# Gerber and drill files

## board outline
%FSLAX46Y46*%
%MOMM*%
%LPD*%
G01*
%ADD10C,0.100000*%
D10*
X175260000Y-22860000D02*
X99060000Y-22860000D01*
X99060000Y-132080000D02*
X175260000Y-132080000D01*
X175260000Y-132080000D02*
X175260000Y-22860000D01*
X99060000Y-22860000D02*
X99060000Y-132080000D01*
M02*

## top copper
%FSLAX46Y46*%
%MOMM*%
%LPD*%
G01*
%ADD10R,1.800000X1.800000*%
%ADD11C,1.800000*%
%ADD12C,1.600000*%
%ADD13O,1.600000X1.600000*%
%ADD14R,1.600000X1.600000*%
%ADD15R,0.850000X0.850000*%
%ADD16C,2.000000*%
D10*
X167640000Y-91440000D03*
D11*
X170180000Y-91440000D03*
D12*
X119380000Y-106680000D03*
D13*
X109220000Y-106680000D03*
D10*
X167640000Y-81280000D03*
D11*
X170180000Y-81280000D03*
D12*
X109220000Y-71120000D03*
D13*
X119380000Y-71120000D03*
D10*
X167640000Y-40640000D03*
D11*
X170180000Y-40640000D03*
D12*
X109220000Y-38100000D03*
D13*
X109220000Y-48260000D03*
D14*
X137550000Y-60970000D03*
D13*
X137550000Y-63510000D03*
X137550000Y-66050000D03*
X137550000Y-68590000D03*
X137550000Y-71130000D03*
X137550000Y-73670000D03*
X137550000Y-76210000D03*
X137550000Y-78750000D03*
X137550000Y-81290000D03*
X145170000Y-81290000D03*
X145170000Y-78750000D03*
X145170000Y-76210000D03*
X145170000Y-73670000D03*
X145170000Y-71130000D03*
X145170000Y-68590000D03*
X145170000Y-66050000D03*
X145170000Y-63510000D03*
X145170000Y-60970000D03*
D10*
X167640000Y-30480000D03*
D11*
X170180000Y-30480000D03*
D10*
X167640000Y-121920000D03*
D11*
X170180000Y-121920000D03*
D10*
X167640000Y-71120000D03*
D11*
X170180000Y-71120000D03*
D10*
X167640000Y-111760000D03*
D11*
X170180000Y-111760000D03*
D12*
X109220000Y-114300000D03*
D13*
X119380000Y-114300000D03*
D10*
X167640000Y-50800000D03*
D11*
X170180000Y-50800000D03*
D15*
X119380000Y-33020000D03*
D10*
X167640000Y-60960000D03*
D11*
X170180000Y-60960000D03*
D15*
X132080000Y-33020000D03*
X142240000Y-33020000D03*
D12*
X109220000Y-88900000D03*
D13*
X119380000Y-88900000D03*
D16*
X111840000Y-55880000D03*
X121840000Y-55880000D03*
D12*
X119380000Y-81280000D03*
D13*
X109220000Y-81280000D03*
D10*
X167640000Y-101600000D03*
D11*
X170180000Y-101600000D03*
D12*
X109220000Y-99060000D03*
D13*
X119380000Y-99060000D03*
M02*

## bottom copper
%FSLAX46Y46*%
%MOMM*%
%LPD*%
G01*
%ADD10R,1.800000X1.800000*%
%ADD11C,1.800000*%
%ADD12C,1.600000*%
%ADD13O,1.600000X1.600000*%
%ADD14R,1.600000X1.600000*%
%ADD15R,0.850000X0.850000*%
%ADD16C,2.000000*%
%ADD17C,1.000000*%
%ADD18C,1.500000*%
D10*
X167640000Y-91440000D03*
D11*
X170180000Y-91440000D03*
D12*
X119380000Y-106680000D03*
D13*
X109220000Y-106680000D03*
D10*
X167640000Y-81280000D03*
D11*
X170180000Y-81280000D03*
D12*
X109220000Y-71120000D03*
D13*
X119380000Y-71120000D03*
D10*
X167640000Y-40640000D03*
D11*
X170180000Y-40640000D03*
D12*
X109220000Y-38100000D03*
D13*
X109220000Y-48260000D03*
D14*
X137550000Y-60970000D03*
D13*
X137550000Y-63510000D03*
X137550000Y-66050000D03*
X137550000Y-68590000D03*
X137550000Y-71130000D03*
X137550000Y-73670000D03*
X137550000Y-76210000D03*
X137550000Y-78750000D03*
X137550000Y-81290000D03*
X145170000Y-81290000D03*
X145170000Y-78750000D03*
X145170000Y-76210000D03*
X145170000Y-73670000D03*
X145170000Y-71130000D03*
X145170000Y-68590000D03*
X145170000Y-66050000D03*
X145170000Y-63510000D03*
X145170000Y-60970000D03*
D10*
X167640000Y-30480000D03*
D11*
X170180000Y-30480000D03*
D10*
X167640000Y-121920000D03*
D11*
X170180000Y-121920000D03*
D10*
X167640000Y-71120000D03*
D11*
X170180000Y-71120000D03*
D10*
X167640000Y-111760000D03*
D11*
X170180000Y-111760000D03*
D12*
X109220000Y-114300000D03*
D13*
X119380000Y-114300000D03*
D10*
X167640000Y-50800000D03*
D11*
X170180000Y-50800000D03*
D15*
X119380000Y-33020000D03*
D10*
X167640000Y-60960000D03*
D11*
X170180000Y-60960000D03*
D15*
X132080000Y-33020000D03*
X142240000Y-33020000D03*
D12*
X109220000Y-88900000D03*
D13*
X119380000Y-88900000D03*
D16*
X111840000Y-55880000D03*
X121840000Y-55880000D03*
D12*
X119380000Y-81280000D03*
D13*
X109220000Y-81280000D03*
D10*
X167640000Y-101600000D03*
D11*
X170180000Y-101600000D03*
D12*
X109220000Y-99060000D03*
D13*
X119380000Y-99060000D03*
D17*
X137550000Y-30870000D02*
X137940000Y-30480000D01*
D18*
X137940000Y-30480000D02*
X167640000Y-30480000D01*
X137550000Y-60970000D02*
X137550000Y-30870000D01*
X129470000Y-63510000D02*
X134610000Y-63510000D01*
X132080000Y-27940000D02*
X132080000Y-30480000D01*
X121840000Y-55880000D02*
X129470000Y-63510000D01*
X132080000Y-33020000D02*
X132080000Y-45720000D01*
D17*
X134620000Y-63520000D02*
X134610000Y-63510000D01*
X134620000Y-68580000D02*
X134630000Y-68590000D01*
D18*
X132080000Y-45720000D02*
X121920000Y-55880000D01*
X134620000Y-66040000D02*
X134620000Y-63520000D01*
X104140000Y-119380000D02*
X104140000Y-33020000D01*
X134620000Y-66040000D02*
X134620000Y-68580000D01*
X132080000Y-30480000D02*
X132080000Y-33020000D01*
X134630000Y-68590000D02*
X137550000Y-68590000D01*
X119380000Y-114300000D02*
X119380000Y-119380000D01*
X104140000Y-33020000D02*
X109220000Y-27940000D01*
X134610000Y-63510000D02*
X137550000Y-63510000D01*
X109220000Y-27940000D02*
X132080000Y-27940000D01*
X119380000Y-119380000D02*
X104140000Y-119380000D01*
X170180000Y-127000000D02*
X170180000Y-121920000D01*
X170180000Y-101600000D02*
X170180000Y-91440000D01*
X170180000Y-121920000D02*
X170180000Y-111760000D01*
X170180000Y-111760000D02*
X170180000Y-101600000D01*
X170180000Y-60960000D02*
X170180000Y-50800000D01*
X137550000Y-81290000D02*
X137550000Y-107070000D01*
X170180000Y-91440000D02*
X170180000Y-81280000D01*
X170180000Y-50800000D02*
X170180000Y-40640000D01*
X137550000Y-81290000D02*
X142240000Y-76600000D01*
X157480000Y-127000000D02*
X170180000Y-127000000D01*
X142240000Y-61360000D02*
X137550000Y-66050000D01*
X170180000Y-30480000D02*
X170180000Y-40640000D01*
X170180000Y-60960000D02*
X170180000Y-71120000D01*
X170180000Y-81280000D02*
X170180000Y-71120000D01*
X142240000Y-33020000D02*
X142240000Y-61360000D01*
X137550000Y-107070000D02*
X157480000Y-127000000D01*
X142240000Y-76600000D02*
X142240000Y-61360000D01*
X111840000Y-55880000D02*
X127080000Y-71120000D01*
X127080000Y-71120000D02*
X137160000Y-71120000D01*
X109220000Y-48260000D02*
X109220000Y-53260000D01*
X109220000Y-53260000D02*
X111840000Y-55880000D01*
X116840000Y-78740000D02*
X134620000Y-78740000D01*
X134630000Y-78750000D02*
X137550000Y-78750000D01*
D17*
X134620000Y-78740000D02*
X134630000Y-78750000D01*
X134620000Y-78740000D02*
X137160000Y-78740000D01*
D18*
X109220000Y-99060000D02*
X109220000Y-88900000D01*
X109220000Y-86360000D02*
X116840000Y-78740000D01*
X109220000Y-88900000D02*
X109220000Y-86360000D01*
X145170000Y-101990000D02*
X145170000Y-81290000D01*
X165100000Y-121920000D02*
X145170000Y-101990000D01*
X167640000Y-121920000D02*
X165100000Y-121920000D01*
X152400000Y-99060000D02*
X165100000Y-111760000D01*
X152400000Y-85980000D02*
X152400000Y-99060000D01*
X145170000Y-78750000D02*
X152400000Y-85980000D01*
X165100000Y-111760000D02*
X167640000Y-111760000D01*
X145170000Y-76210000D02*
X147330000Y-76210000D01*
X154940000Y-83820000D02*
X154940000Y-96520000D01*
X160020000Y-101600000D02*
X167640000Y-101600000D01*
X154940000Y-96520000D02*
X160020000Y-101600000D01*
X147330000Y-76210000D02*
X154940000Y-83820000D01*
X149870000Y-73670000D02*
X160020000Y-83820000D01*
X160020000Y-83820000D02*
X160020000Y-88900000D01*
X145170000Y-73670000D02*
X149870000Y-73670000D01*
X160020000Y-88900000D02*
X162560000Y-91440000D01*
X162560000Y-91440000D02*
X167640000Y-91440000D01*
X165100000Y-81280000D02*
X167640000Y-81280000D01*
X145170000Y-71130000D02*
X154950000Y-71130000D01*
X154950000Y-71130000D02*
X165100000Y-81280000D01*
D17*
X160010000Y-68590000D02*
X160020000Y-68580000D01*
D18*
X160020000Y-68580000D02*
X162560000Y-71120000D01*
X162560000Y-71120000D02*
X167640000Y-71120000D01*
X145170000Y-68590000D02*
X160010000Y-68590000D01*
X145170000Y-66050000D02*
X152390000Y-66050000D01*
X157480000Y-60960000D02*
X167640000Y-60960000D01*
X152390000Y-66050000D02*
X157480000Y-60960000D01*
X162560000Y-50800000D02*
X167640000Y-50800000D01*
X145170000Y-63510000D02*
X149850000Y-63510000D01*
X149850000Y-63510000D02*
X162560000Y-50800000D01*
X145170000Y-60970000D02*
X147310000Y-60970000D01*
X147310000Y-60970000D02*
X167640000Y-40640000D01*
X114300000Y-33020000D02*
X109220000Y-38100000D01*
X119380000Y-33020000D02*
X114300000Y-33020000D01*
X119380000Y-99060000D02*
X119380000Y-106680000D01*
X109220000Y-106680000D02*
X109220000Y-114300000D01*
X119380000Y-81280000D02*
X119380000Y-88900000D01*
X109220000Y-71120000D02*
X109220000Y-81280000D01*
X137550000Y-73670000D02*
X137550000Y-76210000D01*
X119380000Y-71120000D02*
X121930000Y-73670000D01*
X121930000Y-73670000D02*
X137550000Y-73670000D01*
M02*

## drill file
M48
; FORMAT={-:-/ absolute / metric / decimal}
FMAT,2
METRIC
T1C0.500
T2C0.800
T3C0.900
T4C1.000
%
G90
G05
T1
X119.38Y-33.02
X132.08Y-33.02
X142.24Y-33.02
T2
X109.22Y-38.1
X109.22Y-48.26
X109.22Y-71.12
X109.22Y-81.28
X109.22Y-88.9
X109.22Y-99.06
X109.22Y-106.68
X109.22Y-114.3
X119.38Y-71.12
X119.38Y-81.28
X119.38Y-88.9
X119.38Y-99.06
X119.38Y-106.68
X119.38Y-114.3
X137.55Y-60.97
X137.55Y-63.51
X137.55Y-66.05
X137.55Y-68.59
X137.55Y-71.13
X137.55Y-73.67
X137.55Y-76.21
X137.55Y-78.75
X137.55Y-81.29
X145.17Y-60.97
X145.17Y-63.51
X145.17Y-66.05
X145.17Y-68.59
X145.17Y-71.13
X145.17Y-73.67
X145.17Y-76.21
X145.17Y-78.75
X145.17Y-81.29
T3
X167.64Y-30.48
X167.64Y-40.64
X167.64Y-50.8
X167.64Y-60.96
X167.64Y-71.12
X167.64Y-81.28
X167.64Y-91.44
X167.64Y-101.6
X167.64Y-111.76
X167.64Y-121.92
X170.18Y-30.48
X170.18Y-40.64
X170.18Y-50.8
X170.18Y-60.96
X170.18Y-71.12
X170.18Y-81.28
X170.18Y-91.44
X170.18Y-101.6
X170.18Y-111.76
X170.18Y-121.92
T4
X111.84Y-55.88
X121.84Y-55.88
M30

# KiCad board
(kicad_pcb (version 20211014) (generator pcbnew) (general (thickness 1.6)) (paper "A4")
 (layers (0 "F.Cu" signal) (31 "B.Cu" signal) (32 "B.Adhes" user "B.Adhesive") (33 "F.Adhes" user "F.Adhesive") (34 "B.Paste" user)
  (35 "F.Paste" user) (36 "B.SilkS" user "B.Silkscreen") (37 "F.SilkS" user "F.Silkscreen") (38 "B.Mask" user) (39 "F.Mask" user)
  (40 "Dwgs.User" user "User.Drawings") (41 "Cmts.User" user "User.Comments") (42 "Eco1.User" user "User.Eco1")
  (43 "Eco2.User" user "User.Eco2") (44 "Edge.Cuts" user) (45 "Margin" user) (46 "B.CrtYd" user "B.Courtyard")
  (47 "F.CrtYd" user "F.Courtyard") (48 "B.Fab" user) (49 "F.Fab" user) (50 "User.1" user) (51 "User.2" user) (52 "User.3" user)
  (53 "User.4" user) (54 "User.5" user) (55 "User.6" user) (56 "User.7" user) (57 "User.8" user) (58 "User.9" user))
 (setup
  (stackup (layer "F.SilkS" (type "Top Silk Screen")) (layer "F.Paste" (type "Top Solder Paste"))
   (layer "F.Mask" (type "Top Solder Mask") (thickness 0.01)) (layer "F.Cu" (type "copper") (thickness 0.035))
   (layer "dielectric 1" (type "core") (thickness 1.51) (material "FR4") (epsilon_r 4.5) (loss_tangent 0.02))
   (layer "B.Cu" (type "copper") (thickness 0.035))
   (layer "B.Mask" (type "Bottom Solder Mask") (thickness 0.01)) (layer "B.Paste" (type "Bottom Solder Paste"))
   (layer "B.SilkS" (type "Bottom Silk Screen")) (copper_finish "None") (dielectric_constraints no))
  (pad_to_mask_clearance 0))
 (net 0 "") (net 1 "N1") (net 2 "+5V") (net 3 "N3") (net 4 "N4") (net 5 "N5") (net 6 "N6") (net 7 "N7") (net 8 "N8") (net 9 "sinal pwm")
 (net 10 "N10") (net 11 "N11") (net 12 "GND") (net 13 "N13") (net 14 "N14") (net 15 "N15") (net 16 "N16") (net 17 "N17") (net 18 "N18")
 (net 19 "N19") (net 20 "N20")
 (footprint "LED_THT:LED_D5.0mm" (layer "F.Cu") (at 167.64 91.44)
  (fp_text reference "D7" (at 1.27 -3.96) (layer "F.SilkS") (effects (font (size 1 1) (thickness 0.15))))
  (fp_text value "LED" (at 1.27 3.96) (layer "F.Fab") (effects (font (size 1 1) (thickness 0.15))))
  (pad "1" thru_hole rect (at 0 0) (size 1.8 1.8) (drill 0.9) (layers *.Cu *.Mask) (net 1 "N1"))
  (pad "2" thru_hole circle (at 2.54 0) (size 1.8 1.8) (drill 0.9) (layers *.Cu *.Mask) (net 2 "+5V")))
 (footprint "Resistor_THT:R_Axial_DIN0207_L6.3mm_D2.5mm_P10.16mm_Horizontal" (layer "F.Cu") (at 119.38 106.68 180)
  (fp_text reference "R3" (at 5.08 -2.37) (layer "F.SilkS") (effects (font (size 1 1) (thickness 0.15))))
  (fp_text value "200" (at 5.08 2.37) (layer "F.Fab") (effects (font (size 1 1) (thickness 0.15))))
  (pad "1" thru_hole circle (at 0 0 180) (size 1.6 1.6) (drill 0.8) (layers *.Cu *.Mask) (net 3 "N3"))
  (pad "2" thru_hole oval (at 10.16 0 180) (size 1.6 1.6) (drill 0.8) (layers *.Cu *.Mask) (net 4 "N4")))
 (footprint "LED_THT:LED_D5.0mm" (layer "F.Cu") (at 167.64 81.28)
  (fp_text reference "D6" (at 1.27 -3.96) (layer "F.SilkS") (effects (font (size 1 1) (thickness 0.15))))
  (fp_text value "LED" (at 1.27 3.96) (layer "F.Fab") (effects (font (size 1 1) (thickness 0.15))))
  (pad "1" thru_hole rect (at 0 0) (size 1.8 1.8) (drill 0.9) (layers *.Cu *.Mask) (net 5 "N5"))
  (pad "2" thru_hole circle (at 2.54 0) (size 1.8 1.8) (drill 0.9) (layers *.Cu *.Mask) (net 2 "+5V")))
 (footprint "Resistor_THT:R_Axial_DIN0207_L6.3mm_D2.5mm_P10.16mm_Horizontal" (layer "F.Cu") (at 109.22 71.12)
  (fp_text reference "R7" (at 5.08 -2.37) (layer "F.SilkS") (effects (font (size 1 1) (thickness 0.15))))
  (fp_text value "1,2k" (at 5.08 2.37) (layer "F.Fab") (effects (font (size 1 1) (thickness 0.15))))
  (pad "1" thru_hole circle (at 0 0) (size 1.6 1.6) (drill 0.8) (layers *.Cu *.Mask) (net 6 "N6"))
  (pad "2" thru_hole oval (at 10.16 0) (size 1.6 1.6) (drill 0.8) (layers *.Cu *.Mask) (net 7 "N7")))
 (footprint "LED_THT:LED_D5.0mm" (layer "F.Cu") (at 167.64 40.64)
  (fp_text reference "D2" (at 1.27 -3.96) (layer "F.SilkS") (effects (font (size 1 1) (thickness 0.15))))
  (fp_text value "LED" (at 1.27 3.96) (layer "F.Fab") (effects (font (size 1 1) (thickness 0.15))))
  (pad "1" thru_hole rect (at 0 0) (size 1.8 1.8) (drill 0.9) (layers *.Cu *.Mask) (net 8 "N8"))
  (pad "2" thru_hole circle (at 2.54 0) (size 1.8 1.8) (drill 0.9) (layers *.Cu *.Mask) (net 2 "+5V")))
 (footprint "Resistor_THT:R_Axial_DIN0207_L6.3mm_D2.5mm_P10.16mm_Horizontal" (layer "F.Cu") (at 109.22 38.1 -90)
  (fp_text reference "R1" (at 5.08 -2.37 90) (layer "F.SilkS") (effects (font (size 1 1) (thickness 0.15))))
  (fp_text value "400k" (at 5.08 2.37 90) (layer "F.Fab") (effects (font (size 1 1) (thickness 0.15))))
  (pad "1" thru_hole circle (at 0 0 270) (size 1.6 1.6) (drill 0.8) (layers *.Cu *.Mask) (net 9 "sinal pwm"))
  (pad "2" thru_hole oval (at 10.16 0 270) (size 1.6 1.6) (drill 0.8) (layers *.Cu *.Mask) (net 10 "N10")))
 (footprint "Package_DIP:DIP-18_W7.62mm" (layer "F.Cu") (at 137.55 60.97)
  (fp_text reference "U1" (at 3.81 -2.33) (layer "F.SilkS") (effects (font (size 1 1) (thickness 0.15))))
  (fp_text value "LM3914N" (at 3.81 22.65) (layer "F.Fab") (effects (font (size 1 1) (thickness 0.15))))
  (pad "1" thru_hole rect (at 0 0) (size 1.6 1.6) (drill 0.8) (layers *.Cu *.Mask) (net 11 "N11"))
  (pad "2" thru_hole oval (at 0 2.54) (size 1.6 1.6) (drill 0.8) (layers *.Cu *.Mask) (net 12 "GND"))
  (pad "3" thru_hole oval (at 0 5.08) (size 1.6 1.6) (drill 0.8) (layers *.Cu *.Mask) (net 2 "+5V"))
  (pad "4" thru_hole oval (at 0 7.62) (size 1.6 1.6) (drill 0.8) (layers *.Cu *.Mask) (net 12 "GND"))
  (pad "5" thru_hole oval (at 0 10.16) (size 1.6 1.6) (drill 0.8) (layers *.Cu *.Mask) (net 10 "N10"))
  (pad "6" thru_hole oval (at 0 12.7) (size 1.6 1.6) (drill 0.8) (layers *.Cu *.Mask) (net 7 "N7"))
  (pad "7" thru_hole oval (at 0 15.24) (size 1.6 1.6) (drill 0.8) (layers *.Cu *.Mask) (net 7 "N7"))
  (pad "8" thru_hole oval (at 0 17.78) (size 1.6 1.6) (drill 0.8) (layers *.Cu *.Mask) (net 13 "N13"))
  (pad "9" thru_hole oval (at 0 20.32) (size 1.6 1.6) (drill 0.8) (layers *.Cu *.Mask) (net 2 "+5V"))
  (pad "10" thru_hole oval (at 7.62 20.32) (size 1.6 1.6) (drill 0.8) (layers *.Cu *.Mask) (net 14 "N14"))
  (pad "11" thru_hole oval (at 7.62 17.78) (size 1.6 1.6) (drill 0.8) (layers *.Cu *.Mask) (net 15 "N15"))
  (pad "12" thru_hole oval (at 7.62 15.24) (size 1.6 1.6) (drill 0.8) (layers *.Cu *.Mask) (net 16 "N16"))
  (pad "13" thru_hole oval (at 7.62 12.7) (size 1.6 1.6) (drill 0.8) (layers *.Cu *.Mask) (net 1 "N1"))
  (pad "14" thru_hole oval (at 7.62 10.16) (size 1.6 1.6) (drill 0.8) (layers *.Cu *.Mask) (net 5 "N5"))
  (pad "15" thru_hole oval (at 7.62 7.62) (size 1.6 1.6) (drill 0.8) (layers *.Cu *.Mask) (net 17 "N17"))
  (pad "16" thru_hole oval (at 7.62 5.08) (size 1.6 1.6) (drill 0.8) (layers *.Cu *.Mask) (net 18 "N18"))
  (pad "17" thru_hole oval (at 7.62 2.54) (size 1.6 1.6) (drill 0.8) (layers *.Cu *.Mask) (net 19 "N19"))
  (pad "18" thru_hole oval (at 7.62 0) (size 1.6 1.6) (drill 0.8) (layers *.Cu *.Mask) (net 8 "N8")))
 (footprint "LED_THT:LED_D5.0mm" (layer "F.Cu") (at 167.64 30.48)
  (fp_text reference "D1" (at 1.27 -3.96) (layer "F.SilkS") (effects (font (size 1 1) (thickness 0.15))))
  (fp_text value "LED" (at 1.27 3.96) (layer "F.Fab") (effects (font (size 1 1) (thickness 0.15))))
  (pad "1" thru_hole rect (at 0 0) (size 1.8 1.8) (drill 0.9) (layers *.Cu *.Mask) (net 11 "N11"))
  (pad "2" thru_hole circle (at 2.54 0) (size 1.8 1.8) (drill 0.9) (layers *.Cu *.Mask) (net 2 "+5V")))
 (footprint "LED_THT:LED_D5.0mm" (layer "F.Cu") (at 167.64 121.92)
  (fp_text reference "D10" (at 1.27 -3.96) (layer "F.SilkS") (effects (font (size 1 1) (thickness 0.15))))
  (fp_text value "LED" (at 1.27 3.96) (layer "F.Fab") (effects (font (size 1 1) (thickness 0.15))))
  (pad "1" thru_hole rect (at 0 0) (size 1.8 1.8) (drill 0.9) (layers *.Cu *.Mask) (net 14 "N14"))
  (pad "2" thru_hole circle (at 2.54 0) (size 1.8 1.8) (drill 0.9) (layers *.Cu *.Mask) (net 2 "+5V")))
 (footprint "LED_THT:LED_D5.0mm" (layer "F.Cu") (at 167.64 71.12)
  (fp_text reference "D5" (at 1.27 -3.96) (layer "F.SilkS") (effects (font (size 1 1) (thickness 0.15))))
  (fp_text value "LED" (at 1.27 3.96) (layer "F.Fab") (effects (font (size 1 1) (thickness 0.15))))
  (pad "1" thru_hole rect (at 0 0) (size 1.8 1.8) (drill 0.9) (layers *.Cu *.Mask) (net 17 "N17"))
  (pad "2" thru_hole circle (at 2.54 0) (size 1.8 1.8) (drill 0.9) (layers *.Cu *.Mask) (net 2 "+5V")))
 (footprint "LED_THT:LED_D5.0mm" (layer "F.Cu") (at 167.64 111.76)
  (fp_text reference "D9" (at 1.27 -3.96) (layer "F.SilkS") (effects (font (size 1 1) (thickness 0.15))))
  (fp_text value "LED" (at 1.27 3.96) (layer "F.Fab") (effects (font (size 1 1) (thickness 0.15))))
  (pad "1" thru_hole rect (at 0 0) (size 1.8 1.8) (drill 0.9) (layers *.Cu *.Mask) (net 15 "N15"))
  (pad "2" thru_hole circle (at 2.54 0) (size 1.8 1.8) (drill 0.9) (layers *.Cu *.Mask) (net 2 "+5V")))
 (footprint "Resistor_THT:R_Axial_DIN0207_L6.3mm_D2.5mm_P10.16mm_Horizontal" (layer "F.Cu") (at 109.22 114.3)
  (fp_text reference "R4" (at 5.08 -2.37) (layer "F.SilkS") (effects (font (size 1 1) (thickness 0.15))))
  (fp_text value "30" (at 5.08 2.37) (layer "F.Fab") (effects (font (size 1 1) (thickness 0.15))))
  (pad "1" thru_hole circle (at 0 0) (size 1.6 1.6) (drill 0.8) (layers *.Cu *.Mask) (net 4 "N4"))
  (pad "2" thru_hole oval (at 10.16 0) (size 1.6 1.6) (drill 0.8) (layers *.Cu *.Mask) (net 12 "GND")))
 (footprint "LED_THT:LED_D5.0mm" (layer "F.Cu") (at 167.64 50.8)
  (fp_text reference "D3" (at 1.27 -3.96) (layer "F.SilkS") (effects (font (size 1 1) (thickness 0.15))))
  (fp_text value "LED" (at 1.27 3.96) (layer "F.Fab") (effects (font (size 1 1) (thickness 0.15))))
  (pad "1" thru_hole rect (at 0 0) (size 1.8 1.8) (drill 0.9) (layers *.Cu *.Mask) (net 19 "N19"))
  (pad "2" thru_hole circle (at 2.54 0) (size 1.8 1.8) (drill 0.9) (layers *.Cu *.Mask) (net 2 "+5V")))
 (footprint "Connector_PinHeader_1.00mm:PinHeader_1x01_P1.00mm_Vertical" (layer "F.Cu") (at 119.38 33.02)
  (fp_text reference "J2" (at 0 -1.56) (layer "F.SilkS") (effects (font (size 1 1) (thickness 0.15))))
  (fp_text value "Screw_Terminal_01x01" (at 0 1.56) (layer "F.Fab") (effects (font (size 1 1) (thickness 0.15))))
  (pad "1" thru_hole rect (at 0 0) (size 0.85 0.85) (drill 0.5) (layers *.Cu *.Mask) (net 9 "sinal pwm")))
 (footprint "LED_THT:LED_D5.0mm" (layer "F.Cu") (at 167.64 60.96)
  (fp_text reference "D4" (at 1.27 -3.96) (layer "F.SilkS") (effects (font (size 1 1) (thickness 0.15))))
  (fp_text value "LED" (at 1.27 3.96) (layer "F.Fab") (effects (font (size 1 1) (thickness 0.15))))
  (pad "1" thru_hole rect (at 0 0) (size 1.8 1.8) (drill 0.9) (layers *.Cu *.Mask) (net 18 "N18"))
  (pad "2" thru_hole circle (at 2.54 0) (size 1.8 1.8) (drill 0.9) (layers *.Cu *.Mask) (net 2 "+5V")))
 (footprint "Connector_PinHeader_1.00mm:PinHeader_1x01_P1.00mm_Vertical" (layer "F.Cu") (at 132.08 33.02)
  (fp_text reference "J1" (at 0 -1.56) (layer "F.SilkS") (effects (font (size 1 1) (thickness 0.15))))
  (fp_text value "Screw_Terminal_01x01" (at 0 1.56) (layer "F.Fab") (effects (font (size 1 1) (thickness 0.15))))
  (pad "1" thru_hole rect (at 0 0) (size 0.85 0.85) (drill 0.5) (layers *.Cu *.Mask) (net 12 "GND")))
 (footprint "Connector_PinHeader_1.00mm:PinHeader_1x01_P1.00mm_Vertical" (layer "F.Cu") (at 142.24 33.02)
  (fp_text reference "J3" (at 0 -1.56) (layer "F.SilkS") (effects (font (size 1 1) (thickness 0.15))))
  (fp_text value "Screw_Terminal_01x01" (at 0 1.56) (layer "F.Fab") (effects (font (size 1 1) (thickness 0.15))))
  (pad "1" thru_hole rect (at 0 0) (size 0.85 0.85) (drill 0.5) (layers *.Cu *.Mask) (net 2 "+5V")))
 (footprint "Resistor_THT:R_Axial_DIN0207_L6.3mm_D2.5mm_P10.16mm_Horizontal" (layer "F.Cu") (at 109.22 88.9)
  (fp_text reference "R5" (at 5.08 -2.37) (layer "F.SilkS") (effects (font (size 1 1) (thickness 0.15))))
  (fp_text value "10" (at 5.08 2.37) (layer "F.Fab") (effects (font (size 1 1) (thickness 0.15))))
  (pad "1" thru_hole circle (at 0 0) (size 1.6 1.6) (drill 0.8) (layers *.Cu *.Mask) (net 13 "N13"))
  (pad "2" thru_hole oval (at 10.16 0) (size 1.6 1.6) (drill 0.8) (layers *.Cu *.Mask) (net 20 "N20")))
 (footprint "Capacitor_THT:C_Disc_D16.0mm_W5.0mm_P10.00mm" (layer "F.Cu") (at 111.84 55.88)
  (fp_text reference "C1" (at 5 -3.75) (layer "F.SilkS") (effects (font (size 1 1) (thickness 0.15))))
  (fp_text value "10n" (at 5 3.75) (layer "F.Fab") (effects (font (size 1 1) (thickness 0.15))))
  (pad "1" thru_hole circle (at 0 0) (size 2 2) (drill 1) (layers *.Cu *.Mask) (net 10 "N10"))
  (pad "2" thru_hole circle (at 10 0) (size 2 2) (drill 1) (layers *.Cu *.Mask) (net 12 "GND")))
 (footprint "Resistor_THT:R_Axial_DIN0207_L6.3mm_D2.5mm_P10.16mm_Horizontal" (layer "F.Cu") (at 119.38 81.28 180)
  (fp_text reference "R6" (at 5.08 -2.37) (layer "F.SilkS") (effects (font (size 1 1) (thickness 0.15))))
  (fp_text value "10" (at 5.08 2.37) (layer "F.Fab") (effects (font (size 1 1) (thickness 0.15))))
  (pad "1" thru_hole circle (at 0 0 180) (size 1.6 1.6) (drill 0.8) (layers *.Cu *.Mask) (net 20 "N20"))
  (pad "2" thru_hole oval (at 10.16 0 180) (size 1.6 1.6) (drill 0.8) (layers *.Cu *.Mask) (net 6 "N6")))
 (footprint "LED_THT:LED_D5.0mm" (layer "F.Cu") (at 167.64 101.6)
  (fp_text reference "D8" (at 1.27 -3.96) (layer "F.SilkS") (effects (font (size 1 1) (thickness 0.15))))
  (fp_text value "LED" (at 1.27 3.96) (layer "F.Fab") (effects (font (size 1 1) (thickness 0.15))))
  (pad "1" thru_hole rect (at 0 0) (size 1.8 1.8) (drill 0.9) (layers *.Cu *.Mask) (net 16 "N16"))
  (pad "2" thru_hole circle (at 2.54 0) (size 1.8 1.8) (drill 0.9) (layers *.Cu *.Mask) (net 2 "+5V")))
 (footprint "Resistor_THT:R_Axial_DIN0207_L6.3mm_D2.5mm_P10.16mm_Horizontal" (layer "F.Cu") (at 109.22 99.06)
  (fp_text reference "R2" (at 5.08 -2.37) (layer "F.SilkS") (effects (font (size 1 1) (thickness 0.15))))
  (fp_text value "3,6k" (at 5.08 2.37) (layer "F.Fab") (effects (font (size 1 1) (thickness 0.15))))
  (pad "1" thru_hole circle (at 0 0) (size 1.6 1.6) (drill 0.8) (layers *.Cu *.Mask) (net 13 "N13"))
  (pad "2" thru_hole oval (at 10.16 0) (size 1.6 1.6) (drill 0.8) (layers *.Cu *.Mask) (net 3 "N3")))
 (gr_rect (start 177.8 134.62) (end 177.8 134.62) (layer "B.Cu") (width 0.2) (fill none))
 (gr_line (start 175.26 22.86) (end 99.06 22.86) (layer "Edge.Cuts") (width 0.1))
 (gr_line (start 99.06 132.08) (end 175.26 132.08) (layer "Edge.Cuts") (width 0.1))
 (gr_line (start 175.26 132.08) (end 175.26 22.86) (layer "Edge.Cuts") (width 0.1))
 (gr_line (start 99.06 22.86) (end 99.06 132.08) (layer "Edge.Cuts") (width 0.1))
 (segment (start 137.55 30.87) (end 137.94 30.48) (width 1) (layer "B.Cu") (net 11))
 (segment (start 137.94 30.48) (end 167.64 30.48) (width 1.5) (layer "B.Cu") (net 11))
 (segment (start 137.55 60.97) (end 137.55 30.87) (width 1.5) (layer "B.Cu") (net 11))
 (segment (start 129.47 63.51) (end 134.61 63.51) (width 1.5) (layer "B.Cu") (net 12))
 (segment (start 132.08 27.94) (end 132.08 30.48) (width 1.5) (layer "B.Cu") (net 12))
 (segment (start 121.84 55.88) (end 129.47 63.51) (width 1.5) (layer "B.Cu") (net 12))
 (segment (start 132.08 33.02) (end 132.08 45.72) (width 1.5) (layer "B.Cu") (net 12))
 (segment (start 134.62 63.52) (end 134.61 63.51) (width 1) (layer "B.Cu") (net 12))
 (segment (start 134.62 68.58) (end 134.63 68.59) (width 1) (layer "B.Cu") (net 12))
 (segment (start 132.08 45.72) (end 121.92 55.88) (width 1.5) (layer "B.Cu") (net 12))
 (segment (start 134.62 66.04) (end 134.62 63.52) (width 1.5) (layer "B.Cu") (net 12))
 (segment (start 104.14 119.38) (end 104.14 33.02) (width 1.5) (layer "B.Cu") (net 12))
 (segment (start 134.62 66.04) (end 134.62 68.58) (width 1.5) (layer "B.Cu") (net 12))
 (segment (start 132.08 30.48) (end 132.08 33.02) (width 1.5) (layer "B.Cu") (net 12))
 (segment (start 134.63 68.59) (end 137.55 68.59) (width 1.5) (layer "B.Cu") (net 12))
 (segment (start 119.38 114.3) (end 119.38 119.38) (width 1.5) (layer "B.Cu") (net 12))
 (segment (start 104.14 33.02) (end 109.22 27.94) (width 1.5) (layer "B.Cu") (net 12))
 (segment (start 134.61 63.51) (end 137.55 63.51) (width 1.5) (layer "B.Cu") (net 12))
 (segment (start 109.22 27.94) (end 132.08 27.94) (width 1.5) (layer "B.Cu") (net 12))
 (segment (start 119.38 119.38) (end 104.14 119.38) (width 1.5) (layer "B.Cu") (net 12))
 (segment (start 170.18 127) (end 170.18 121.92) (width 1.5) (layer "B.Cu") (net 2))
 (segment (start 170.18 101.6) (end 170.18 91.44) (width 1.5) (layer "B.Cu") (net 2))
 (segment (start 170.18 121.92) (end 170.18 111.76) (width 1.5) (layer "B.Cu") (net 2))
 (segment (start 170.18 111.76) (end 170.18 101.6) (width 1.5) (layer "B.Cu") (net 2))
 (segment (start 170.18 60.96) (end 170.18 50.8) (width 1.5) (layer "B.Cu") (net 2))
 (segment (start 137.55 81.29) (end 137.55 107.07) (width 1.5) (layer "B.Cu") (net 2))
 (segment (start 170.18 91.44) (end 170.18 81.28) (width 1.5) (layer "B.Cu") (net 2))
 (segment (start 170.18 50.8) (end 170.18 40.64) (width 1.5) (layer "B.Cu") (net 2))
 (segment (start 137.55 81.29) (end 142.24 76.6) (width 1.5) (layer "B.Cu") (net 2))
 (segment (start 157.48 127) (end 170.18 127) (width 1.5) (layer "B.Cu") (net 2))
 (segment (start 142.24 61.36) (end 137.55 66.05) (width 1.5) (layer "B.Cu") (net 2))
 (segment (start 170.18 30.48) (end 170.18 40.64) (width 1.5) (layer "B.Cu") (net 2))
 (segment (start 170.18 60.96) (end 170.18 71.12) (width 1.5) (layer "B.Cu") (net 2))
 (segment (start 170.18 81.28) (end 170.18 71.12) (width 1.5) (layer "B.Cu") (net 2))
 (segment (start 142.24 33.02) (end 142.24 61.36) (width 1.5) (layer "B.Cu") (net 2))
 (segment (start 137.55 107.07) (end 157.48 127) (width 1.5) (layer "B.Cu") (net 2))
 (segment (start 142.24 76.6) (end 142.24 61.36) (width 1.5) (layer "B.Cu") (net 2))
 (segment (start 111.84 55.88) (end 127.08 71.12) (width 1.5) (layer "B.Cu") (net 10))
 (segment (start 127.08 71.12) (end 137.16 71.12) (width 1.5) (layer "B.Cu") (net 10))
 (segment (start 109.22 48.26) (end 109.22 53.26) (width 1.5) (layer "B.Cu") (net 10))
 (segment (start 109.22 53.26) (end 111.84 55.88) (width 1.5) (layer "B.Cu") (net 10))
 (segment (start 116.84 78.74) (end 134.62 78.74) (width 1.5) (layer "B.Cu") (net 13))
 (segment (start 134.63 78.75) (end 137.55 78.75) (width 1.5) (layer "B.Cu") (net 13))
 (segment (start 134.62 78.74) (end 134.63 78.75) (width 1) (layer "B.Cu") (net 13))
 (segment (start 134.62 78.74) (end 137.16 78.74) (width 1) (layer "B.Cu") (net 13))
 (segment (start 109.22 99.06) (end 109.22 88.9) (width 1.5) (layer "B.Cu") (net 13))
 (segment (start 109.22 86.36) (end 116.84 78.74) (width 1.5) (layer "B.Cu") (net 13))
 (segment (start 109.22 88.9) (end 109.22 86.36) (width 1.5) (layer "B.Cu") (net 13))
 (segment (start 145.17 101.99) (end 145.17 81.29) (width 1.5) (layer "B.Cu") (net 14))
 (segment (start 165.1 121.92) (end 145.17 101.99) (width 1.5) (layer "B.Cu") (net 14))
 (segment (start 167.64 121.92) (end 165.1 121.92) (width 1.5) (layer "B.Cu") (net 14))
 (segment (start 152.4 99.06) (end 165.1 111.76) (width 1.5) (layer "B.Cu") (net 15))
 (segment (start 152.4 85.98) (end 152.4 99.06) (width 1.5) (layer "B.Cu") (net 15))
 (segment (start 145.17 78.75) (end 152.4 85.98) (width 1.5) (layer "B.Cu") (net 15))
 (segment (start 165.1 111.76) (end 167.64 111.76) (width 1.5) (layer "B.Cu") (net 15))
 (segment (start 145.17 76.21) (end 147.33 76.21) (width 1.5) (layer "B.Cu") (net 16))
 (segment (start 154.94 83.82) (end 154.94 96.52) (width 1.5) (layer "B.Cu") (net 16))
 (segment (start 160.02 101.6) (end 167.64 101.6) (width 1.5) (layer "B.Cu") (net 16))
 (segment (start 154.94 96.52) (end 160.02 101.6) (width 1.5) (layer "B.Cu") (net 16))
 (segment (start 147.33 76.21) (end 154.94 83.82) (width 1.5) (layer "B.Cu") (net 16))
 (segment (start 149.87 73.67) (end 160.02 83.82) (width 1.5) (layer "B.Cu") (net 1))
 (segment (start 160.02 83.82) (end 160.02 88.9) (width 1.5) (layer "B.Cu") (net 1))
 (segment (start 145.17 73.67) (end 149.87 73.67) (width 1.5) (layer "B.Cu") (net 1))
 (segment (start 160.02 88.9) (end 162.56 91.44) (width 1.5) (layer "B.Cu") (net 1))
 (segment (start 162.56 91.44) (end 167.64 91.44) (width 1.5) (layer "B.Cu") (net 1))
 (segment (start 165.1 81.28) (end 167.64 81.28) (width 1.5) (layer "B.Cu") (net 5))
 (segment (start 145.17 71.13) (end 154.95 71.13) (width 1.5) (layer "B.Cu") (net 5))
 (segment (start 154.95 71.13) (end 165.1 81.28) (width 1.5) (layer "B.Cu") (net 5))
 (segment (start 160.01 68.59) (end 160.02 68.58) (width 1) (layer "B.Cu") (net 17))
 (segment (start 160.02 68.58) (end 162.56 71.12) (width 1.5) (layer "B.Cu") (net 17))
 (segment (start 162.56 71.12) (end 167.64 71.12) (width 1.5) (layer "B.Cu") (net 17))
 (segment (start 145.17 68.59) (end 160.01 68.59) (width 1.5) (layer "B.Cu") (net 17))
 (segment (start 145.17 66.05) (end 152.39 66.05) (width 1.5) (layer "B.Cu") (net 18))
 (segment (start 157.48 60.96) (end 167.64 60.96) (width 1.5) (layer "B.Cu") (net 18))
 (segment (start 152.39 66.05) (end 157.48 60.96) (width 1.5) (layer "B.Cu") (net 18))
 (segment (start 162.56 50.8) (end 167.64 50.8) (width 1.5) (layer "B.Cu") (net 19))
 (segment (start 145.17 63.51) (end 149.85 63.51) (width 1.5) (layer "B.Cu") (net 19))
 (segment (start 149.85 63.51) (end 162.56 50.8) (width 1.5) (layer "B.Cu") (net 19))
 (segment (start 145.17 60.97) (end 147.31 60.97) (width 1.5) (layer "B.Cu") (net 8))
 (segment (start 147.31 60.97) (end 167.64 40.64) (width 1.5) (layer "B.Cu") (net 8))
 (segment (start 114.3 33.02) (end 109.22 38.1) (width 1.5) (layer "B.Cu") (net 9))
 (segment (start 119.38 33.02) (end 114.3 33.02) (width 1.5) (layer "B.Cu") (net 9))
 (segment (start 119.38 99.06) (end 119.38 106.68) (width 1.5) (layer "B.Cu") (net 3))
 (segment (start 109.22 106.68) (end 109.22 114.3) (width 1.5) (layer "B.Cu") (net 4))
 (segment (start 119.38 81.28) (end 119.38 88.9) (width 1.5) (layer "B.Cu") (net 20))
 (segment (start 109.22 71.12) (end 109.22 81.28) (width 1.5) (layer "B.Cu") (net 6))
 (segment (start 137.55 73.67) (end 137.55 76.21) (width 1.5) (layer "B.Cu") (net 7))
 (segment (start 119.38 71.12) (end 121.93 73.67) (width 1.5) (layer "B.Cu") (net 7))
 (segment (start 121.93 73.67) (end 137.55 73.67) (width 1.5) (layer "B.Cu") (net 7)))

